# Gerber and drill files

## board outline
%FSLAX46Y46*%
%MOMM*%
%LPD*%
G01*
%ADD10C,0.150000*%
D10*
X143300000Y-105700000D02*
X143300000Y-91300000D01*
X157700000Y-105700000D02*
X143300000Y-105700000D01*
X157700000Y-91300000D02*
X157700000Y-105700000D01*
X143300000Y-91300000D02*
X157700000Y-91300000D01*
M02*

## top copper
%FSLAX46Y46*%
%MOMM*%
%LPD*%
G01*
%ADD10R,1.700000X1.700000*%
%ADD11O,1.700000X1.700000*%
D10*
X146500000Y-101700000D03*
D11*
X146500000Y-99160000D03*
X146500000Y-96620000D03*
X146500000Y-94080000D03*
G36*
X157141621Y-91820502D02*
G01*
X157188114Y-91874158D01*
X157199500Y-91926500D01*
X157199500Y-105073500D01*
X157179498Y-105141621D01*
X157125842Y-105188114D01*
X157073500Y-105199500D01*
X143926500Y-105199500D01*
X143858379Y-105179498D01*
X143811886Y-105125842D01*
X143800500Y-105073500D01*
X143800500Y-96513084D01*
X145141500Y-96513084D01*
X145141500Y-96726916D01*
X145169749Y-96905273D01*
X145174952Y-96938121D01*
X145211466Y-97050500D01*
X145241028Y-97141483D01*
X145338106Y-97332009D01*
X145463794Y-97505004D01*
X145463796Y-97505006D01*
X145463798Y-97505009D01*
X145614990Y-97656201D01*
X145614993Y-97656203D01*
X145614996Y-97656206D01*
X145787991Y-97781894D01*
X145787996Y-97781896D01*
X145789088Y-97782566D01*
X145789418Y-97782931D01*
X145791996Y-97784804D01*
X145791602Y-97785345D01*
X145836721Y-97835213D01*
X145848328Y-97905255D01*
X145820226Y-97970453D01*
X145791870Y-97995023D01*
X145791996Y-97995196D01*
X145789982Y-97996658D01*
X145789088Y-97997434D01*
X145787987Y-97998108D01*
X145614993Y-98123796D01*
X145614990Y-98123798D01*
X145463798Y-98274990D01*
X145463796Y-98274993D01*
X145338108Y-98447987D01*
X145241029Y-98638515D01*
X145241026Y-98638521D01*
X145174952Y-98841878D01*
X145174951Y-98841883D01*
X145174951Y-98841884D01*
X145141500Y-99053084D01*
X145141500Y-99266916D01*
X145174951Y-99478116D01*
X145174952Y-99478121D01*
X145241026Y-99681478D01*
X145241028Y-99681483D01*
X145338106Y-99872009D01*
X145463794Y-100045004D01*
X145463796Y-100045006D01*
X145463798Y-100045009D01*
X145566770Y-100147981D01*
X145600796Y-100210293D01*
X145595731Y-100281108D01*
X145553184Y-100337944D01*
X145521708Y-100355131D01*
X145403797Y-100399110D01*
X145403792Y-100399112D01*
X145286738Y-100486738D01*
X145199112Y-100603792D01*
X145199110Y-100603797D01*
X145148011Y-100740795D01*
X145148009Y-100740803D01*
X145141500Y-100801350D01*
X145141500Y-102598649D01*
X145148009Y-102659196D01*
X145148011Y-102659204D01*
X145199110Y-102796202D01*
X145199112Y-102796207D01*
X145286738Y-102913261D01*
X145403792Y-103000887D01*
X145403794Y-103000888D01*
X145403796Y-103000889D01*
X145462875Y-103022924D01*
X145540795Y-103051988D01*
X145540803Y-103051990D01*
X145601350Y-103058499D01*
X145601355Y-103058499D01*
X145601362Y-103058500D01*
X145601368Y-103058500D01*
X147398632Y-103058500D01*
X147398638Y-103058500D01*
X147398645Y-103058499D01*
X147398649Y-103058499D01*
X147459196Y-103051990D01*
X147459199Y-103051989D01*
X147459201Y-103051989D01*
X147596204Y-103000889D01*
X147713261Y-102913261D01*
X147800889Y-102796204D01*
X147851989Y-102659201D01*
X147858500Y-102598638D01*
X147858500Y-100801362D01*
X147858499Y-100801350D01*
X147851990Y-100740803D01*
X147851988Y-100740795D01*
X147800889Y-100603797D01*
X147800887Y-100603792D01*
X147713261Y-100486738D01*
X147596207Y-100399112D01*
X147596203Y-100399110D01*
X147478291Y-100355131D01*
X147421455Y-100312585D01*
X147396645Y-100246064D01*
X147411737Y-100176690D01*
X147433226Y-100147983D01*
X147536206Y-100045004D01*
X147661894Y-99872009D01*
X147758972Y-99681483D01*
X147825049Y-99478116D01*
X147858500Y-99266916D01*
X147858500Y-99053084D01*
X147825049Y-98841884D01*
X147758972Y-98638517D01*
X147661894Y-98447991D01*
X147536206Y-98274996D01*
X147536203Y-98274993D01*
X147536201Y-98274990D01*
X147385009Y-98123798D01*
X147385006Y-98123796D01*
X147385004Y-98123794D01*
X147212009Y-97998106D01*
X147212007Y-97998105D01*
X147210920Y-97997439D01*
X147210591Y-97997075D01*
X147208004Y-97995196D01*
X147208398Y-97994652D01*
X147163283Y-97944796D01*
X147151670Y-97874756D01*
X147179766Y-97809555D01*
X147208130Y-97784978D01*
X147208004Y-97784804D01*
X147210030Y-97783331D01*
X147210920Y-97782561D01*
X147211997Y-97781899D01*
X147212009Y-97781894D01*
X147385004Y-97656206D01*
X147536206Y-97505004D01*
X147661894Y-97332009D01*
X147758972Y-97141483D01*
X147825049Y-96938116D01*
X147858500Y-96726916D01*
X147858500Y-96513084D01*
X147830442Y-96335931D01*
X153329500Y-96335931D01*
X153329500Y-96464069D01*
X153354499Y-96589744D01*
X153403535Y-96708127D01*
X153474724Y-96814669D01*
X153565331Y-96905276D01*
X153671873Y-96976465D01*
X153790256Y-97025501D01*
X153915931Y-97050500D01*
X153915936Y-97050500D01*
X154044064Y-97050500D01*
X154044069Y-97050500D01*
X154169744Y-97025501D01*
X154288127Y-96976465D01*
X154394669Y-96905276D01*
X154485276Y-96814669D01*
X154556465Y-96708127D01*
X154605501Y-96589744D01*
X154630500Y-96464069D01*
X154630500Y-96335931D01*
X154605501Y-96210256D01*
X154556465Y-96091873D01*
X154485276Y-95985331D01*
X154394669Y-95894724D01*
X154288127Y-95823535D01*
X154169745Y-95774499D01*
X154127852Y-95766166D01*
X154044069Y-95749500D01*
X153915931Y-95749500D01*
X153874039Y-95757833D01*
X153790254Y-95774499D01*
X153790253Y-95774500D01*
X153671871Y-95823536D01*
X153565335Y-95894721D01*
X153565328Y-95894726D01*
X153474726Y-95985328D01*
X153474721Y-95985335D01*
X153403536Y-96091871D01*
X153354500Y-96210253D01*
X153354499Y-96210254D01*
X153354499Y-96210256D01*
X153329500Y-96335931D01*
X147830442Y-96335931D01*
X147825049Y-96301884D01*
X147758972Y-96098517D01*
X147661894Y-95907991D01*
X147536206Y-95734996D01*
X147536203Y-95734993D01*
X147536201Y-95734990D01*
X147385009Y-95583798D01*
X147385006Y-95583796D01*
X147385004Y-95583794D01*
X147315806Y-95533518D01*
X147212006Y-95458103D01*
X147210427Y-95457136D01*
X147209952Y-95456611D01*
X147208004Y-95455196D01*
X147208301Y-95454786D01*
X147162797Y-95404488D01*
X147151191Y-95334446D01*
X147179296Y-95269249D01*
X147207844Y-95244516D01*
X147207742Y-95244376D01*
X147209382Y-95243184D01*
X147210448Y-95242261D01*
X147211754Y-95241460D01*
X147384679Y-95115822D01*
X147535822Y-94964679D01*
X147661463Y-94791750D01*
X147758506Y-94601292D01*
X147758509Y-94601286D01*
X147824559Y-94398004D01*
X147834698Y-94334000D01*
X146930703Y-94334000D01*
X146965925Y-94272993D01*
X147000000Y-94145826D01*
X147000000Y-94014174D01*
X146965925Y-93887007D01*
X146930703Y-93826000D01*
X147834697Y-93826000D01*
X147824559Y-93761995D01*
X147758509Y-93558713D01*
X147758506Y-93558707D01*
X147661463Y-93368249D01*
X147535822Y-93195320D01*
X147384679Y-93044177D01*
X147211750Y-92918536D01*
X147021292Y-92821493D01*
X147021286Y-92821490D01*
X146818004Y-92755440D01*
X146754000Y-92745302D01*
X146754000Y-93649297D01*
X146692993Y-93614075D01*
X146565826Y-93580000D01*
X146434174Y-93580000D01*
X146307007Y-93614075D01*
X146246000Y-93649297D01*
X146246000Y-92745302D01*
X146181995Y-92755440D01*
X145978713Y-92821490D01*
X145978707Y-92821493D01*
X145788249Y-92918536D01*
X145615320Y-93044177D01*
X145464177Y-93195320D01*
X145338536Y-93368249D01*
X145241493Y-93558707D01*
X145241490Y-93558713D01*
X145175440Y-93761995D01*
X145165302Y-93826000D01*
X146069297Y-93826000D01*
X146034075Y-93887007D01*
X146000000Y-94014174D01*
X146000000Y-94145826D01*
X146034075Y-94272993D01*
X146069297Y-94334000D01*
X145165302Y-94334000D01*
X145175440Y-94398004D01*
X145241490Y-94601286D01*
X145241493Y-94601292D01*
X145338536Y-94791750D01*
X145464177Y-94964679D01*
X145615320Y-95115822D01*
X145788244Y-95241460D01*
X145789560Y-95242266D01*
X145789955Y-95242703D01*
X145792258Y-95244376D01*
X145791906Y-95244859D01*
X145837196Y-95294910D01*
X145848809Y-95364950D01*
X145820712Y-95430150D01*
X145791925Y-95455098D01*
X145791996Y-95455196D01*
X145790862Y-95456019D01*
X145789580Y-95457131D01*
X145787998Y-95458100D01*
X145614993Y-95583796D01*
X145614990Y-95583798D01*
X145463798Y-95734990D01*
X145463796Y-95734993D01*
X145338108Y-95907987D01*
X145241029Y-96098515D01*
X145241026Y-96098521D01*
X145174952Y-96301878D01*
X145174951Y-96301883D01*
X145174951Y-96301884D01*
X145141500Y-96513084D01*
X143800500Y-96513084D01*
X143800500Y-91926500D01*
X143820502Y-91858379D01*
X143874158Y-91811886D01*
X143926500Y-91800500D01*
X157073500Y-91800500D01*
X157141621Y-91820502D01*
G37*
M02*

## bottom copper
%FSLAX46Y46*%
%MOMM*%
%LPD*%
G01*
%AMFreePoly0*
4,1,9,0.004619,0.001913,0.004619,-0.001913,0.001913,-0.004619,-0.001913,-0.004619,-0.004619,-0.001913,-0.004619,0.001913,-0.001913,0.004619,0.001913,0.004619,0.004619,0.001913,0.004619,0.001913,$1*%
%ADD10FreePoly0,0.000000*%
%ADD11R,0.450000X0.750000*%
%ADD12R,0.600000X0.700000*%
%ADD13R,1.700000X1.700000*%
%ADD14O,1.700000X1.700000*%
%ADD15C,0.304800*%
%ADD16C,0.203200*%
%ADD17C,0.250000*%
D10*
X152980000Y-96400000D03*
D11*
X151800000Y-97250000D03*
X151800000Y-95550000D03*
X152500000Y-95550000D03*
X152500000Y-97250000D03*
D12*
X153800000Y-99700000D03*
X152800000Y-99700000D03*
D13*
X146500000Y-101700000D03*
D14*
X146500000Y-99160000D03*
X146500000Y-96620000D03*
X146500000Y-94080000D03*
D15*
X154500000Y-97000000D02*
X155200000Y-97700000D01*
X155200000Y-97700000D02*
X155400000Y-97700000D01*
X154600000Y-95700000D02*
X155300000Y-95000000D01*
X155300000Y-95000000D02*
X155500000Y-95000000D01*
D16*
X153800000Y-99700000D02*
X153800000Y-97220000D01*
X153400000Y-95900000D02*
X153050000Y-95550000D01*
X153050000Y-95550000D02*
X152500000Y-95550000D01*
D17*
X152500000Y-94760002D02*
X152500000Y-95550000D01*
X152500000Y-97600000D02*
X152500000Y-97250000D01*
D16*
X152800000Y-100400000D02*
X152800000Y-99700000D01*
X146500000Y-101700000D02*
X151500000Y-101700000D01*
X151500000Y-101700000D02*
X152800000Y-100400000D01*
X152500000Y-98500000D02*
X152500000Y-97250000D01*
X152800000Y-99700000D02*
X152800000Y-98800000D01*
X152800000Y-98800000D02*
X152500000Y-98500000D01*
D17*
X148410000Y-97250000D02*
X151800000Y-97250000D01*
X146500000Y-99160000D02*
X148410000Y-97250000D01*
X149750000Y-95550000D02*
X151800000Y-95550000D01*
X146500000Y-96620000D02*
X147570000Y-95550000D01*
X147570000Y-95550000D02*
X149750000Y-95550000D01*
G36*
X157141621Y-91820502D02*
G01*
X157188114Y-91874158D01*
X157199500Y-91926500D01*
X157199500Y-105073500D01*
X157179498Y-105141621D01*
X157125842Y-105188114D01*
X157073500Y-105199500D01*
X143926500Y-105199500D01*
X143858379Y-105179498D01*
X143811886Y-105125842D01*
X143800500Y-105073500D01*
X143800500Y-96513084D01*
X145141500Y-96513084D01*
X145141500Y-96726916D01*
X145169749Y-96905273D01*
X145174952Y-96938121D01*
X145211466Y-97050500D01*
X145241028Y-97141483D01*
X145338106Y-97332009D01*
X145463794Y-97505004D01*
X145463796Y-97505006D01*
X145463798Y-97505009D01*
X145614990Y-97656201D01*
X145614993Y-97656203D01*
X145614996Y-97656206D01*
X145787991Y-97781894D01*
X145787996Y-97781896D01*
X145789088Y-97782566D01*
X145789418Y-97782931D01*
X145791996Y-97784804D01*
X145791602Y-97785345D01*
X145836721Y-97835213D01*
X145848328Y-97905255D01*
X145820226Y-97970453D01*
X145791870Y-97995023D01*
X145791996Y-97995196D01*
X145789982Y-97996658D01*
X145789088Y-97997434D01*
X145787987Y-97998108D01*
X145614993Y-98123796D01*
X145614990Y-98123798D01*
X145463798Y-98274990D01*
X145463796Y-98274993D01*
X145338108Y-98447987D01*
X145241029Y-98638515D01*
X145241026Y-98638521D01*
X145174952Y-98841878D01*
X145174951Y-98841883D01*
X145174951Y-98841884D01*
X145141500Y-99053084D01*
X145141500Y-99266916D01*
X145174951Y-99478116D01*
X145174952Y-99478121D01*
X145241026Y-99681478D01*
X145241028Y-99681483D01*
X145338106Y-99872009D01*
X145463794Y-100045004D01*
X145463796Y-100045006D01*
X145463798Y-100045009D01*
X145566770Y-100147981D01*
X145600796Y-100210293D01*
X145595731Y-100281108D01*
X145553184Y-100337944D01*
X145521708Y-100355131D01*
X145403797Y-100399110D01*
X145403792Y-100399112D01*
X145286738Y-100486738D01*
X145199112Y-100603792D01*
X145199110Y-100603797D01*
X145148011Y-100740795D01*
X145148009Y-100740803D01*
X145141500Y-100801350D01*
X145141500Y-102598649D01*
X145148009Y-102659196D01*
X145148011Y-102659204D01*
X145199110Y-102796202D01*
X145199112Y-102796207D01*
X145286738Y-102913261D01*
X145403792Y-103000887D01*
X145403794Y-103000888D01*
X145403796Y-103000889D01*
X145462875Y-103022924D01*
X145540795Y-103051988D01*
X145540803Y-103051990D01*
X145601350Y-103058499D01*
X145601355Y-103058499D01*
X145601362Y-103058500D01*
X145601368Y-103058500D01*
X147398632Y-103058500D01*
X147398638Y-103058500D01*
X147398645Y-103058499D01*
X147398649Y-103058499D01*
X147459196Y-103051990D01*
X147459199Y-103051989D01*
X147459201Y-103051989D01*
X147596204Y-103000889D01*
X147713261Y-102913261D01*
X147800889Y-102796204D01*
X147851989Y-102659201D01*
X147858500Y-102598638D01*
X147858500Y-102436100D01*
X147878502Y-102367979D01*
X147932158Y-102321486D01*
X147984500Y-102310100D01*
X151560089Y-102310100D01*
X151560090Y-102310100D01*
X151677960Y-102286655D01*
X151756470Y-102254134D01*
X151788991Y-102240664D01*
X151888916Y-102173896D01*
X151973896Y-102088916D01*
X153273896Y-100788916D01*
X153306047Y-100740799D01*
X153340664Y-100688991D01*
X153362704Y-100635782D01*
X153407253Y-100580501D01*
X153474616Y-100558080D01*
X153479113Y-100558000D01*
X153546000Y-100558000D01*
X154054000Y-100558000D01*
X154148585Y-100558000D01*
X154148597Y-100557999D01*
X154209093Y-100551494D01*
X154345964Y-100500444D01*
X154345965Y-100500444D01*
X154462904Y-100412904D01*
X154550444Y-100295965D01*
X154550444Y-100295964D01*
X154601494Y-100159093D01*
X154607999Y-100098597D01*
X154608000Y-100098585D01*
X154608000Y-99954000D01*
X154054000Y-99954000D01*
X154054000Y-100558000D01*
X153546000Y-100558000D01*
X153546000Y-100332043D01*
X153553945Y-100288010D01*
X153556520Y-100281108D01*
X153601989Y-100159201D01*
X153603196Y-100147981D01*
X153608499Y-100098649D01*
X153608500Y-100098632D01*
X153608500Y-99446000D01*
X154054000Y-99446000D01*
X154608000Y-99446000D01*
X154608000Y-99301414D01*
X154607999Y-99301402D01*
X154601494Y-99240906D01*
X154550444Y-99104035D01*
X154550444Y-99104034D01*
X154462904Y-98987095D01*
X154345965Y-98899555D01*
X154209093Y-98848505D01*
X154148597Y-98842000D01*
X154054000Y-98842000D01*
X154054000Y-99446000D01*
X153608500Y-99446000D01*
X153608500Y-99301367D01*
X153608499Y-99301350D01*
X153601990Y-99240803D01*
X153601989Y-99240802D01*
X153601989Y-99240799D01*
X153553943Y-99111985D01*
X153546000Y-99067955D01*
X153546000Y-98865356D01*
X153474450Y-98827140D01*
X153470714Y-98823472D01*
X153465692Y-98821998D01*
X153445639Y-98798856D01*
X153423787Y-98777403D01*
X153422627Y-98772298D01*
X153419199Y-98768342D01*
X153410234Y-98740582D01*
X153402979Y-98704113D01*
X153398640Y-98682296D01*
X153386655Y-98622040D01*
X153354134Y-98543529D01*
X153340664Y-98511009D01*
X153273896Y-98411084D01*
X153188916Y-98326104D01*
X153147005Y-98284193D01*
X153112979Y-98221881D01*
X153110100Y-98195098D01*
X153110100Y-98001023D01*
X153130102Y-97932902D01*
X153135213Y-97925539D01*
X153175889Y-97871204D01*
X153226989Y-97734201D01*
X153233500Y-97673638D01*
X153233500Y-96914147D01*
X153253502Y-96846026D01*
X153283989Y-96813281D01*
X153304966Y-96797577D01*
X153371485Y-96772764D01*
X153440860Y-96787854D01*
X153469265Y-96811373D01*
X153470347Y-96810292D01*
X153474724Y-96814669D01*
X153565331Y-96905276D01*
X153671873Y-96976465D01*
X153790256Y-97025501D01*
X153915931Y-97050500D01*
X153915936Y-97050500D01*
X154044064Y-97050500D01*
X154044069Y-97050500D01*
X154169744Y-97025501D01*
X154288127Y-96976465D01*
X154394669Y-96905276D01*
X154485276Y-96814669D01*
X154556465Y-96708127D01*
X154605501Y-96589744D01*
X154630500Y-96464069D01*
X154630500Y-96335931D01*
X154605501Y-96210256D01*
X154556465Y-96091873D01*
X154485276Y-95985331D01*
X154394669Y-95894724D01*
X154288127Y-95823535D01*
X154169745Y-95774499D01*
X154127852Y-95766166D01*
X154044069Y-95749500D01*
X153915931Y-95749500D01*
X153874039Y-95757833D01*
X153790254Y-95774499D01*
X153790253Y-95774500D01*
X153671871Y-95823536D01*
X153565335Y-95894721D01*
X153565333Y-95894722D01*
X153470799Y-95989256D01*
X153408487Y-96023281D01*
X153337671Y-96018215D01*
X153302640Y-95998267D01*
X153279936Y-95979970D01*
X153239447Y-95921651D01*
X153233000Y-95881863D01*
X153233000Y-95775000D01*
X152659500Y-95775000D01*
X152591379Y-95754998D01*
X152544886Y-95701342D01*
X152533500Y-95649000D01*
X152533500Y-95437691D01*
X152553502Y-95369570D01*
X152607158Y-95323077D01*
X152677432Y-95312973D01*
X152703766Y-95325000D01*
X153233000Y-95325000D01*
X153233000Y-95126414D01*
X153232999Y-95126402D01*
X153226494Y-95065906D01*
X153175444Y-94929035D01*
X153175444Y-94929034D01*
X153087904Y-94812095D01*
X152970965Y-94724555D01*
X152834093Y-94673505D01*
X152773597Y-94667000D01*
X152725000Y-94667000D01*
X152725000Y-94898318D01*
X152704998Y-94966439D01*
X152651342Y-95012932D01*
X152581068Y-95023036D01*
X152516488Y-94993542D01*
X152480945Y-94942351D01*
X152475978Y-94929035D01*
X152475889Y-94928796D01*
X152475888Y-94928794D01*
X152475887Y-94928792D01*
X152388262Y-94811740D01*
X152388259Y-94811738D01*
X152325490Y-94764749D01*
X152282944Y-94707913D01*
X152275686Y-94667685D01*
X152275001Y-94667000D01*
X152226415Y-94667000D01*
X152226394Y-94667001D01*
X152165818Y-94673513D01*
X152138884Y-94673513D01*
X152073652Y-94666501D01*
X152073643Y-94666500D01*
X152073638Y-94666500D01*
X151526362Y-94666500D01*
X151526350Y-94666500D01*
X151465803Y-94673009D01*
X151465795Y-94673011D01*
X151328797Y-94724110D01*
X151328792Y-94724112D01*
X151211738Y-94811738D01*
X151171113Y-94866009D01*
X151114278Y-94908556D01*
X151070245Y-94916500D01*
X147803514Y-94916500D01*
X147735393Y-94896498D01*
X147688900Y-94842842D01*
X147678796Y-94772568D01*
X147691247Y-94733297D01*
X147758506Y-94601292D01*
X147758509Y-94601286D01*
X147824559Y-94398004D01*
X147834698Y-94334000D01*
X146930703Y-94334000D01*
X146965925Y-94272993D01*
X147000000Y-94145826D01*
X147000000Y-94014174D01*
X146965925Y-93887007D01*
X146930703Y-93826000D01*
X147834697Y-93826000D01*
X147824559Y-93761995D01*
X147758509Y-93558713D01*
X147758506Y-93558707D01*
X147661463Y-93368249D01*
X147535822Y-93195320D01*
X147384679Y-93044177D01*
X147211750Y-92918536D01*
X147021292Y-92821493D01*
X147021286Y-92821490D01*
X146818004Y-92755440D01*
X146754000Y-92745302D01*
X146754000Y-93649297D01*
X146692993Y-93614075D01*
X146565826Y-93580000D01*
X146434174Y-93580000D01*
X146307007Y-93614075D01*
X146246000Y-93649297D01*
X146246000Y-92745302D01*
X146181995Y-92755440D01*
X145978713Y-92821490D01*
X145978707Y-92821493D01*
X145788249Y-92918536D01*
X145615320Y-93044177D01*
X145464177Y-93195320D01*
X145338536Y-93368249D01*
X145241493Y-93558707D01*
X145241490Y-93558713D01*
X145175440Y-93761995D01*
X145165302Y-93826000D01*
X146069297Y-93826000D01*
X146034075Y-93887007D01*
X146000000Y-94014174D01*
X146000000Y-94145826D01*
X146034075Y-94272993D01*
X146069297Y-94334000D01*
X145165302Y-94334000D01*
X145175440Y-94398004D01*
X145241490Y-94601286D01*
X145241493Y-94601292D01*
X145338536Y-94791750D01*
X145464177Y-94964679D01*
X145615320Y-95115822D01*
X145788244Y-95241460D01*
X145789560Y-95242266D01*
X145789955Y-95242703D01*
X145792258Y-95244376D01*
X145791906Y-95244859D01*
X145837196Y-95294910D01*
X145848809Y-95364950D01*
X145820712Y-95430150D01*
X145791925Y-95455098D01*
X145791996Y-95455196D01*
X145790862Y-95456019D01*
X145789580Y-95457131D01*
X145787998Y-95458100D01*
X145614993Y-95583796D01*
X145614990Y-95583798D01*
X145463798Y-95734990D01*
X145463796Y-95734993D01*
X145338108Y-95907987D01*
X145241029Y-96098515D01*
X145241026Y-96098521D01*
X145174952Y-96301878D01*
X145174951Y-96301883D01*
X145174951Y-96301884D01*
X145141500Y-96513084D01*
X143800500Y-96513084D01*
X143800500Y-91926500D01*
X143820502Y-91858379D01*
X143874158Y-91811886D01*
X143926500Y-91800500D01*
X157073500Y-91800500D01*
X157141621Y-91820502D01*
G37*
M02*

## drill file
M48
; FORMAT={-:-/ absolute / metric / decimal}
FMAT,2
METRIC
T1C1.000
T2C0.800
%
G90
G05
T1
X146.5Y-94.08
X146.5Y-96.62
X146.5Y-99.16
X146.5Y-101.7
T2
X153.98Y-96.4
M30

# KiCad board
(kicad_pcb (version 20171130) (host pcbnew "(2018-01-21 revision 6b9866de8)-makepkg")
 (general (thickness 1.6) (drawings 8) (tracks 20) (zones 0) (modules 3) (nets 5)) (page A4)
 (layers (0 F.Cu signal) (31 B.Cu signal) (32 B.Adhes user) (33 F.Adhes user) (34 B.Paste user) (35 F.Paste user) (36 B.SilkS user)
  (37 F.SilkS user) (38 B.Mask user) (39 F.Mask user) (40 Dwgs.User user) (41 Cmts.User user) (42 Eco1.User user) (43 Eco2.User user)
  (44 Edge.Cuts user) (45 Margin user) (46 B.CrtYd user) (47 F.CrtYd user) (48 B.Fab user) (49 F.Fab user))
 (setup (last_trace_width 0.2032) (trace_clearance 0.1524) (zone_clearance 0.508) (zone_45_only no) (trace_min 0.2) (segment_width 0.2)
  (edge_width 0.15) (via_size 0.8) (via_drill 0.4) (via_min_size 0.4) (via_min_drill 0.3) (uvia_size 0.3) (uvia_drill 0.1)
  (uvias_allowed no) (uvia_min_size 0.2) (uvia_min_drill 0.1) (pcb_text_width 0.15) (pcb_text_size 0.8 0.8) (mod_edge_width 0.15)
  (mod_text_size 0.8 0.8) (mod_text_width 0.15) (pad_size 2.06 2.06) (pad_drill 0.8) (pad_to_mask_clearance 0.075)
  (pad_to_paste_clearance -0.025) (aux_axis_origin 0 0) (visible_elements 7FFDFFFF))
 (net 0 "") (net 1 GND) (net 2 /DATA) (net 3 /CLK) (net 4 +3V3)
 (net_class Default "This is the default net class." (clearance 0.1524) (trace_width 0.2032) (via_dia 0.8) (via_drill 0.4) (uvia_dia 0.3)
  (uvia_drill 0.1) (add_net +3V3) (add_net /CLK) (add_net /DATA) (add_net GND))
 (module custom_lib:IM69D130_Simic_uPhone (layer B.Cu) (at 153.3 96.4)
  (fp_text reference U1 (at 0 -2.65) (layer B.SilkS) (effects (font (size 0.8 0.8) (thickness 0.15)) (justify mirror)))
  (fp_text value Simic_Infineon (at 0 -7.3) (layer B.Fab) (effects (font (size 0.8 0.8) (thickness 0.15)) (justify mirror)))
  (pad "" np_thru_hole circle (at 0.68 0) (size 0.8 0.8) (drill 0.8) (layers *.Cu *.Mask) (solder_mask_margin 0.01) (clearance 0.04))
  (pad 5 smd custom (at -0.32 0) (size 0.01 0.01) (layers B.Cu B.Mask) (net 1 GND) (zone_connect 0)
   (options (clearance outline) (anchor circle)) (primitives))
  (pad 1 smd rect (at -1.5 0.85) (size 0.45 0.75) (layers B.Cu B.Paste B.Mask) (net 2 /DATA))
  (pad 3 smd rect (at -1.5 -0.85) (size 0.45 0.75) (layers B.Cu B.Paste B.Mask) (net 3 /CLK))
  (pad 4 smd rect (at -0.8 -0.85) (size 0.45 0.75) (layers B.Cu B.Paste B.Mask) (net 1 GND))
  (pad 2 smd rect (at -0.8 0.85) (size 0.45 0.75) (layers B.Cu B.Paste B.Mask) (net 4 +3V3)))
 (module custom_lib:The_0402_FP (layer B.Cu) (at 153.3 99.7)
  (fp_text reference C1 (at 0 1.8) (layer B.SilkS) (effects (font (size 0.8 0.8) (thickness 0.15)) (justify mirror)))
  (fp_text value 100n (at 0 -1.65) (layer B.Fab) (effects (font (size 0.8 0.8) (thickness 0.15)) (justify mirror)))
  (pad 2 smd rect (at 0.5 0) (size 0.6 0.7) (layers B.Cu B.Paste B.Mask) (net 1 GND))
  (pad 1 smd rect (at -0.5 0) (size 0.6 0.7) (layers B.Cu B.Paste B.Mask) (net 4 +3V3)))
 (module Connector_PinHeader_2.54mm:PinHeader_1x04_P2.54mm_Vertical (layer F.Cu) (at 146.5 101.7 180)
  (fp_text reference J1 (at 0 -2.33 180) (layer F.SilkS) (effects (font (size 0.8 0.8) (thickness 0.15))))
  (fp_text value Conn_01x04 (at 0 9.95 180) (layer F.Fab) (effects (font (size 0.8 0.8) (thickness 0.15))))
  (pad 1 thru_hole rect (at 0 0 180) (size 1.7 1.7) (drill 1) (layers *.Cu *.Mask) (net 4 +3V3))
  (pad 2 thru_hole oval (at 0 2.54 180) (size 1.7 1.7) (drill 1) (layers *.Cu *.Mask) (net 2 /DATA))
  (pad 3 thru_hole oval (at 0 5.08 180) (size 1.7 1.7) (drill 1) (layers *.Cu *.Mask) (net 3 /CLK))
  (pad 4 thru_hole oval (at 0 7.62 180) (size 1.7 1.7) (drill 1) (layers *.Cu *.Mask) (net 1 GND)))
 (gr_line (start 143.3 105.7) (end 143.3 91.3) (layer Edge.Cuts) (width 0.15))
 (gr_line (start 157.7 105.7) (end 143.3 105.7) (layer Edge.Cuts) (width 0.15))
 (gr_line (start 157.7 91.3) (end 157.7 105.7) (layer Edge.Cuts) (width 0.15))
 (gr_line (start 143.3 91.3) (end 157.7 91.3) (layer Edge.Cuts) (width 0.15))
 (segment (start 154.5 97) (end 155.2 97.7) (width 0.3048) (layer B.Cu) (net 1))
 (segment (start 155.2 97.7) (end 155.4 97.7) (width 0.3048) (layer B.Cu) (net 1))
 (segment (start 154.6 95.7) (end 155.3 95) (width 0.3048) (layer B.Cu) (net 1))
 (segment (start 155.3 95) (end 155.5 95) (width 0.3048) (layer B.Cu) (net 1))
 (segment (start 153.8 99.7) (end 153.8 97.22) (width 0.2032) (layer B.Cu) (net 1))
 (segment (start 153.4 95.9) (end 153.05 95.55) (width 0.2032) (layer B.Cu) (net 1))
 (segment (start 153.05 95.55) (end 152.5 95.55) (width 0.2032) (layer B.Cu) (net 1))
 (segment (start 152.5 94.760002) (end 152.5 95.55) (width 0.25) (layer B.Cu) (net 1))
 (segment (start 152.5 97.6) (end 152.5 97.25) (width 0.25) (layer B.Cu) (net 4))
 (segment (start 152.8 100.4) (end 152.8 99.7) (width 0.2032) (layer B.Cu) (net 4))
 (segment (start 146.5 101.7) (end 151.5 101.7) (width 0.2032) (layer B.Cu) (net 4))
 (segment (start 151.5 101.7) (end 152.8 100.4) (width 0.2032) (layer B.Cu) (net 4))
 (segment (start 152.5 98.5) (end 152.5 97.25) (width 0.2032) (layer B.Cu) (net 4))
 (segment (start 152.8 99.7) (end 152.8 98.8) (width 0.2032) (layer B.Cu) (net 4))
 (segment (start 152.8 98.8) (end 152.5 98.5) (width 0.2032) (layer B.Cu) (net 4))
 (segment (start 148.41 97.25) (end 151.8 97.25) (width 0.25) (layer B.Cu) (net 2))
 (segment (start 146.5 99.16) (end 148.41 97.25) (width 0.25) (layer B.Cu) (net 2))
 (segment (start 149.75 95.55) (end 151.8 95.55) (width 0.25) (layer B.Cu) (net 3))
 (segment (start 146.5 96.62) (end 147.57 95.55) (width 0.25) (layer B.Cu) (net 3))
 (segment (start 147.57 95.55) (end 149.75 95.55) (width 0.25) (layer B.Cu) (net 3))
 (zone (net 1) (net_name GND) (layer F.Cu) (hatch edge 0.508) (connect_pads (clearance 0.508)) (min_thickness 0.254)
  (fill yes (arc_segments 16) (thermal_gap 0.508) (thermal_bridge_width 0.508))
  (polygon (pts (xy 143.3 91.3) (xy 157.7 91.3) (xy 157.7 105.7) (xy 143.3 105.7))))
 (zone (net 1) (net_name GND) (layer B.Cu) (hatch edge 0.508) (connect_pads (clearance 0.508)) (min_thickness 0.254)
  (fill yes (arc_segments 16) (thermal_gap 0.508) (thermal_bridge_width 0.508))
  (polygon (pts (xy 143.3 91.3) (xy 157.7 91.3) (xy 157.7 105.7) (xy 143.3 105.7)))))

